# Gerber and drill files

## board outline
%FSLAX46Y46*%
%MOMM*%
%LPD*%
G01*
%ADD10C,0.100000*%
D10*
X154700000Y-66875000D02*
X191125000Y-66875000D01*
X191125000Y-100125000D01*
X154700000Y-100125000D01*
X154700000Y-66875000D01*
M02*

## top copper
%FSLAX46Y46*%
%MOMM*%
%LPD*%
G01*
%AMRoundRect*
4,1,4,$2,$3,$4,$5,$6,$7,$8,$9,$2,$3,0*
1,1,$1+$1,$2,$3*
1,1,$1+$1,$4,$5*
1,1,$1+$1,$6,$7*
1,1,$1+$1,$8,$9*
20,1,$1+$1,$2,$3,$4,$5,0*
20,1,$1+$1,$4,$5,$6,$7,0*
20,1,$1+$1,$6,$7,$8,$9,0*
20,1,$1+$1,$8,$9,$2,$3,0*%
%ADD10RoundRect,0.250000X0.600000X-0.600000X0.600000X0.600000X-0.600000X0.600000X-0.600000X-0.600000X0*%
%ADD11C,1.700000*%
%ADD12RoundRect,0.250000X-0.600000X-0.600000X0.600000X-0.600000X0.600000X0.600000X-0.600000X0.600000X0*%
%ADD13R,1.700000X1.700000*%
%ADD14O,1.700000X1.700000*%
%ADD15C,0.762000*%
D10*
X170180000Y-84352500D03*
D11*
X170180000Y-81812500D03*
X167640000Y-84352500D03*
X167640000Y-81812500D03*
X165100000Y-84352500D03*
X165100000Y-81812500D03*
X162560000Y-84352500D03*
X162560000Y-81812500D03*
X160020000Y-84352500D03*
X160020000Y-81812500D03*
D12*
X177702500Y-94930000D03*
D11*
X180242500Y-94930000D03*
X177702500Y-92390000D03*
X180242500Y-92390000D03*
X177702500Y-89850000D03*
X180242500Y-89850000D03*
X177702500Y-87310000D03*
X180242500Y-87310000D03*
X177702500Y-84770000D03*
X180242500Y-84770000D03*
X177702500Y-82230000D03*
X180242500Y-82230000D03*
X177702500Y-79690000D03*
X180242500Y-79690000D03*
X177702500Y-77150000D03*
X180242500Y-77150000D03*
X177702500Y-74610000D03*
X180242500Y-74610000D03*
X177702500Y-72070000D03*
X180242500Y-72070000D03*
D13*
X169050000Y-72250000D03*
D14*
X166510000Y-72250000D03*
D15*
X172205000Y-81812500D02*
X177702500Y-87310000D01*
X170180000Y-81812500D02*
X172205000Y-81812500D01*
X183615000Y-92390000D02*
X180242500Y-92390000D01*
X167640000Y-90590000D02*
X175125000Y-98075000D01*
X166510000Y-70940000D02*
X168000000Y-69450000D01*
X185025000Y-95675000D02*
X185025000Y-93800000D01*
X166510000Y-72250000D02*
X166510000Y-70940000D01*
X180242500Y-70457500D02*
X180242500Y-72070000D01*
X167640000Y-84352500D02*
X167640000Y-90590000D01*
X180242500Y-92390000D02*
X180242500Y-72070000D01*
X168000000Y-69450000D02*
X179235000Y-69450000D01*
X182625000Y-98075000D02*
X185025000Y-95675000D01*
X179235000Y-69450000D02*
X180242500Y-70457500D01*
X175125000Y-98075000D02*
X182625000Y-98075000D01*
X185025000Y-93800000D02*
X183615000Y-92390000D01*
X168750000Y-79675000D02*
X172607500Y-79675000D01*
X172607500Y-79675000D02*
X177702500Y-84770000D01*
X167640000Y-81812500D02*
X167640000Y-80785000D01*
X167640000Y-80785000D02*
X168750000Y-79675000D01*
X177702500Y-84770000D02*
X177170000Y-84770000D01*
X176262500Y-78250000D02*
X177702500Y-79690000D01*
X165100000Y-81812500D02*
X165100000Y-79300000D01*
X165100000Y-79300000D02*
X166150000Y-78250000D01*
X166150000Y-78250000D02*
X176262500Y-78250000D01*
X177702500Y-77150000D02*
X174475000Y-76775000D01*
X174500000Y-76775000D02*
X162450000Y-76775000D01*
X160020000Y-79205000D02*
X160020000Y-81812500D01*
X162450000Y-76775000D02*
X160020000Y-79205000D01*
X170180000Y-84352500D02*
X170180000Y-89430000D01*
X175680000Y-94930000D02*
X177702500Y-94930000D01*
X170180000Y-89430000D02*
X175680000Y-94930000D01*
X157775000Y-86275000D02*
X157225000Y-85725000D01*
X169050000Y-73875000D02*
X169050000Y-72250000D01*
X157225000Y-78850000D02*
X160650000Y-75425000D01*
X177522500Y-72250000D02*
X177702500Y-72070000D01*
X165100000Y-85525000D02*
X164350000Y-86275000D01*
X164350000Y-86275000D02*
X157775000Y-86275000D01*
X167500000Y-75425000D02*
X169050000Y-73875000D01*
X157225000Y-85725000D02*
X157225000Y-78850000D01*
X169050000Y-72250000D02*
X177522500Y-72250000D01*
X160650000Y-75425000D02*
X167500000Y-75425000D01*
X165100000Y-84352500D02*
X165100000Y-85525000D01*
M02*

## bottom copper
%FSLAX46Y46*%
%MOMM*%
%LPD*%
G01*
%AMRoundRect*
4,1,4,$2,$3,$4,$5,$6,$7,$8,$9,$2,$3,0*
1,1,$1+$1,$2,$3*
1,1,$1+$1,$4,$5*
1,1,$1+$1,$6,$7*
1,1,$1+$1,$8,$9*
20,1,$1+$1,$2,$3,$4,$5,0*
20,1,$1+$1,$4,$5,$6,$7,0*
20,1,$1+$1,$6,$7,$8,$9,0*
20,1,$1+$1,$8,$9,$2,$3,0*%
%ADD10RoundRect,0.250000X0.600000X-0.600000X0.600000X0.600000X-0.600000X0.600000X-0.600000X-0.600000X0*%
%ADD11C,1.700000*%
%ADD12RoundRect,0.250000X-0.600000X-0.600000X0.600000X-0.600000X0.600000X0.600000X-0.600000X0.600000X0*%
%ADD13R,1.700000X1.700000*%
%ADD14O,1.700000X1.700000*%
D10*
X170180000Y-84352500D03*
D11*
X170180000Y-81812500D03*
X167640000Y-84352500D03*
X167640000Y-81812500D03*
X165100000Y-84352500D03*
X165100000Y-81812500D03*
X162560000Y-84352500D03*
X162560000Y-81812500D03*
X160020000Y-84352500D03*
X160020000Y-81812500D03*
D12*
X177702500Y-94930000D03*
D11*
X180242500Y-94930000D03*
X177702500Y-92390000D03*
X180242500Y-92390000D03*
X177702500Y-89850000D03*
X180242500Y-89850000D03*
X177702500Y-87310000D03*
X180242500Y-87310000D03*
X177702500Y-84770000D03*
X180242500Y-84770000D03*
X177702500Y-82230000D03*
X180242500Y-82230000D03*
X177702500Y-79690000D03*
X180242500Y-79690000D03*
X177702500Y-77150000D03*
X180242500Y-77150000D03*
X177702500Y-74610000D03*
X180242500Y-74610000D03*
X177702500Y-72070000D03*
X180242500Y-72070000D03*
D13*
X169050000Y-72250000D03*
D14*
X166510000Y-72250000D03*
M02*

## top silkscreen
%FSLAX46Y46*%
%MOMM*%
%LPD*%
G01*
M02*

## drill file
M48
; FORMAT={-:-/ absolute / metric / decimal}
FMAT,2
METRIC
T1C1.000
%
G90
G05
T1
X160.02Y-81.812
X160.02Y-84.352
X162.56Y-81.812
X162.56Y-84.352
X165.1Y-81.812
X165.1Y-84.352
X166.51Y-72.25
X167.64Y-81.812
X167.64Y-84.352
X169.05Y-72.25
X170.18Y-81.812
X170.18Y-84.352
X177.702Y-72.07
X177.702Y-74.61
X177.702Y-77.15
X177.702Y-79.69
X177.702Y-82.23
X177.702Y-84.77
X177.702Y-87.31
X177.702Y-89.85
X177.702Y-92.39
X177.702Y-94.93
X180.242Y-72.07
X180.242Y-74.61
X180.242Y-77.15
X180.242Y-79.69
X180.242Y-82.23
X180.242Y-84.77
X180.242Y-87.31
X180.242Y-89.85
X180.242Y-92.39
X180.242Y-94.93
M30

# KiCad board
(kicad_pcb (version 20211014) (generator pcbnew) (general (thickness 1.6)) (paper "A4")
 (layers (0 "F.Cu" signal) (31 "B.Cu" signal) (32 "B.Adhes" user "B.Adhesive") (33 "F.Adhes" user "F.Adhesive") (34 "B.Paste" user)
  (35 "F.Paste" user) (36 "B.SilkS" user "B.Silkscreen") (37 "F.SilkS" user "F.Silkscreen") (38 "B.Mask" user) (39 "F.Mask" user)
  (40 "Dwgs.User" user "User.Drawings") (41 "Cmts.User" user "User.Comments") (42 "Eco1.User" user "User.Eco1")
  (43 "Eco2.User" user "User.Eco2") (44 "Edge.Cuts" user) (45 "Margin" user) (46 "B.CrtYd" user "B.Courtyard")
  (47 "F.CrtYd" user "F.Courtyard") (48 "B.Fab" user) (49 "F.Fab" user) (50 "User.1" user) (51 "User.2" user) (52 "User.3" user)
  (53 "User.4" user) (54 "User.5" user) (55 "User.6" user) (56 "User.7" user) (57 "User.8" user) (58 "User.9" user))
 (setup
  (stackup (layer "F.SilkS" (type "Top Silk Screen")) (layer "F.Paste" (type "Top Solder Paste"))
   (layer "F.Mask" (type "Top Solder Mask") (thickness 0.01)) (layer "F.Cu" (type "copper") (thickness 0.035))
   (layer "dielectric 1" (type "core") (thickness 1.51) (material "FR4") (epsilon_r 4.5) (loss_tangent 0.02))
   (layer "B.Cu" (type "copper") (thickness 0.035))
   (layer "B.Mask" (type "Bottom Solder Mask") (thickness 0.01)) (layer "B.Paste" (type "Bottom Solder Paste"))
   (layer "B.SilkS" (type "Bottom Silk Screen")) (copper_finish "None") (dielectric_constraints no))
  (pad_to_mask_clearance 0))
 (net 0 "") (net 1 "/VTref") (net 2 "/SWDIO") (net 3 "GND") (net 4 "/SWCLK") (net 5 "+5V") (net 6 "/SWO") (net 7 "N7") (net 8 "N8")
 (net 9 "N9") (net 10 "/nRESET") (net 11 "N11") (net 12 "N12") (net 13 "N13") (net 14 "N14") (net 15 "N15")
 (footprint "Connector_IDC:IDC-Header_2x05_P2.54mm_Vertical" (layer "B.Cu") (at 170.18 84.3525 90)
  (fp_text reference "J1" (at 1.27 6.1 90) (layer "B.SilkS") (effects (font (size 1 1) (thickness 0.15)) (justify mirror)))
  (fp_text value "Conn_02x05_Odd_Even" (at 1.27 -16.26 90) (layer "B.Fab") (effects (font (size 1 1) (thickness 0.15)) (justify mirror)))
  (pad "1" thru_hole roundrect (at 0 0 90) (size 1.7 1.7) (drill 1) (layers *.Cu *.Mask) (roundrect_rratio 0.147059) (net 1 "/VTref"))
  (pad "2" thru_hole circle (at 2.54 0 90) (size 1.7 1.7) (drill 1) (layers *.Cu *.Mask) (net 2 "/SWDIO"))
  (pad "3" thru_hole circle (at 0 -2.54 90) (size 1.7 1.7) (drill 1) (layers *.Cu *.Mask) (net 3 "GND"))
  (pad "4" thru_hole circle (at 2.54 -2.54 90) (size 1.7 1.7) (drill 1) (layers *.Cu *.Mask) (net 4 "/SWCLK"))
  (pad "5" thru_hole circle (at 0 -5.08 90) (size 1.7 1.7) (drill 1) (layers *.Cu *.Mask) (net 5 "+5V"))
  (pad "6" thru_hole circle (at 2.54 -5.08 90) (size 1.7 1.7) (drill 1) (layers *.Cu *.Mask) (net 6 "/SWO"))
  (pad "7" thru_hole circle (at 0 -7.62 90) (size 1.7 1.7) (drill 1) (layers *.Cu *.Mask) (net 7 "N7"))
  (pad "8" thru_hole circle (at 2.54 -7.62 90) (size 1.7 1.7) (drill 1) (layers *.Cu *.Mask) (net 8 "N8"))
  (pad "9" thru_hole circle (at 0 -10.16 90) (size 1.7 1.7) (drill 1) (layers *.Cu *.Mask) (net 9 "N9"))
  (pad "10" thru_hole circle (at 2.54 -10.16 90) (size 1.7 1.7) (drill 1) (layers *.Cu *.Mask) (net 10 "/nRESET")))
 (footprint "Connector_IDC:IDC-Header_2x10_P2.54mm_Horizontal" (layer "B.Cu") (at 177.7025 94.93)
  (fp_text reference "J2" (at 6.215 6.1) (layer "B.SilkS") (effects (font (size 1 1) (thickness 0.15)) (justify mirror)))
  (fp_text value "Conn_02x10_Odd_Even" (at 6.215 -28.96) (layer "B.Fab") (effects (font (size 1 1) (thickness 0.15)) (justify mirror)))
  (pad "1" thru_hole roundrect (at 0 0) (size 1.7 1.7) (drill 1) (layers *.Cu *.Mask) (roundrect_rratio 0.1470588235) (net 1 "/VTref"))
  (pad "2" thru_hole circle (at 2.54 0) (size 1.7 1.7) (drill 1) (layers *.Cu *.Mask) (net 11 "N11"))
  (pad "3" thru_hole circle (at 0 -2.54) (size 1.7 1.7) (drill 1) (layers *.Cu *.Mask) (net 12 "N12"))
  (pad "4" thru_hole circle (at 2.54 -2.54) (size 1.7 1.7) (drill 1) (layers *.Cu *.Mask) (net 3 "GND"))
  (pad "5" thru_hole circle (at 0 -5.08) (size 1.7 1.7) (drill 1) (layers *.Cu *.Mask) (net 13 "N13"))
  (pad "6" thru_hole circle (at 2.54 -5.08) (size 1.7 1.7) (drill 1) (layers *.Cu *.Mask) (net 3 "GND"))
  (pad "7" thru_hole circle (at 0 -7.62) (size 1.7 1.7) (drill 1) (layers *.Cu *.Mask) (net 2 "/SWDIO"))
  (pad "8" thru_hole circle (at 2.54 -7.62) (size 1.7 1.7) (drill 1) (layers *.Cu *.Mask) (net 3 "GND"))
  (pad "9" thru_hole circle (at 0 -10.16) (size 1.7 1.7) (drill 1) (layers *.Cu *.Mask) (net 4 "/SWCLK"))
  (pad "10" thru_hole circle (at 2.54 -10.16) (size 1.7 1.7) (drill 1) (layers *.Cu *.Mask) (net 3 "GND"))
  (pad "11" thru_hole circle (at 0 -12.7) (size 1.7 1.7) (drill 1) (layers *.Cu *.Mask) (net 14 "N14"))
  (pad "12" thru_hole circle (at 2.54 -12.7) (size 1.7 1.7) (drill 1) (layers *.Cu *.Mask) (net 3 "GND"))
  (pad "13" thru_hole circle (at 0 -15.24) (size 1.7 1.7) (drill 1) (layers *.Cu *.Mask) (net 6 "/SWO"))
  (pad "14" thru_hole circle (at 2.54 -15.24) (size 1.7 1.7) (drill 1) (layers *.Cu *.Mask) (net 3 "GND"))
  (pad "15" thru_hole circle (at 0 -17.78) (size 1.7 1.7) (drill 1) (layers *.Cu *.Mask) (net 10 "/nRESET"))
  (pad "16" thru_hole circle (at 2.54 -17.78) (size 1.7 1.7) (drill 1) (layers *.Cu *.Mask) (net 3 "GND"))
  (pad "17" thru_hole circle (at 0 -20.32) (size 1.7 1.7) (drill 1) (layers *.Cu *.Mask) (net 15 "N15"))
  (pad "18" thru_hole circle (at 2.54 -20.32) (size 1.7 1.7) (drill 1) (layers *.Cu *.Mask) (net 3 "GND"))
  (pad "19" thru_hole circle (at 0 -22.86) (size 1.7 1.7) (drill 1) (layers *.Cu *.Mask) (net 5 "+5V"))
  (pad "20" thru_hole circle (at 2.54 -22.86) (size 1.7 1.7) (drill 1) (layers *.Cu *.Mask) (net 3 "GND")))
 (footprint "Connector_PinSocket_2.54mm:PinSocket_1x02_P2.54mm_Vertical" (layer "B.Cu") (at 169.05 72.25 90)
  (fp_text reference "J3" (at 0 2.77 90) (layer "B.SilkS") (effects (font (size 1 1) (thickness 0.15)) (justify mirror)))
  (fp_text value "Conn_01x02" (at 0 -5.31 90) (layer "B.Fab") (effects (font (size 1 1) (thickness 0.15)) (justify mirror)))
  (pad "1" thru_hole rect (at 0 0 90) (size 1.7 1.7) (drill 1) (layers *.Cu *.Mask) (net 5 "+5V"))
  (pad "2" thru_hole oval (at 0 -2.54 90) (size 1.7 1.7) (drill 1) (layers *.Cu *.Mask) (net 3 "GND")))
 (gr_rect (start 191.125 66.875) (end 154.7 100.125) (layer "Edge.Cuts") (width 0.1) (fill none))
 (segment (start 172.205 81.8125) (end 177.7025 87.31) (width 0.762) (layer "F.Cu") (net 2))
 (segment (start 170.18 81.8125) (end 172.205 81.8125) (width 0.762) (layer "F.Cu") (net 2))
 (segment (start 183.615 92.39) (end 180.2425 92.39) (width 0.762) (layer "F.Cu") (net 3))
 (segment (start 167.64 90.59) (end 175.125 98.075) (width 0.762) (layer "F.Cu") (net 3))
 (segment (start 166.51 70.94) (end 168 69.45) (width 0.762) (layer "F.Cu") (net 3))
 (segment (start 185.025 95.675) (end 185.025 93.8) (width 0.762) (layer "F.Cu") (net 3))
 (segment (start 166.51 72.25) (end 166.51 70.94) (width 0.762) (layer "F.Cu") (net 3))
 (segment (start 180.2425 70.4575) (end 180.2425 72.07) (width 0.762) (layer "F.Cu") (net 3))
 (segment (start 167.64 84.3525) (end 167.64 90.59) (width 0.762) (layer "F.Cu") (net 3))
 (segment (start 180.2425 92.39) (end 180.2425 72.07) (width 0.762) (layer "F.Cu") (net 3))
 (segment (start 168 69.45) (end 179.235 69.45) (width 0.762) (layer "F.Cu") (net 3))
 (segment (start 182.625 98.075) (end 185.025 95.675) (width 0.762) (layer "F.Cu") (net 3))
 (segment (start 179.235 69.45) (end 180.2425 70.4575) (width 0.762) (layer "F.Cu") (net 3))
 (segment (start 175.125 98.075) (end 182.625 98.075) (width 0.762) (layer "F.Cu") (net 3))
 (segment (start 185.025 93.8) (end 183.615 92.39) (width 0.762) (layer "F.Cu") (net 3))
 (segment (start 168.75 79.675) (end 172.6075 79.675) (width 0.762) (layer "F.Cu") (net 4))
 (segment (start 172.6075 79.675) (end 177.7025 84.77) (width 0.762) (layer "F.Cu") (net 4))
 (segment (start 167.64 81.8125) (end 167.64 80.785) (width 0.762) (layer "F.Cu") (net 4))
 (segment (start 167.64 80.785) (end 168.75 79.675) (width 0.762) (layer "F.Cu") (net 4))
 (segment (start 177.7025 84.77) (end 177.17 84.77) (width 0.762) (layer "F.Cu") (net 4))
 (segment (start 176.2625 78.25) (end 177.7025 79.69) (width 0.762) (layer "F.Cu") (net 6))
 (segment (start 165.1 81.8125) (end 165.1 79.3) (width 0.762) (layer "F.Cu") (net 6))
 (segment (start 165.1 79.3) (end 166.15 78.25) (width 0.762) (layer "F.Cu") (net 6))
 (segment (start 166.15 78.25) (end 176.2625 78.25) (width 0.762) (layer "F.Cu") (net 6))
 (segment (start 177.7025 77.15) (end 174.475 76.775) (width 0.762) (layer "F.Cu") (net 10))
 (segment (start 174.5 76.775) (end 162.45 76.775) (width 0.762) (layer "F.Cu") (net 10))
 (segment (start 160.02 79.205) (end 160.02 81.8125) (width 0.762) (layer "F.Cu") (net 10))
 (segment (start 162.45 76.775) (end 160.02 79.205) (width 0.762) (layer "F.Cu") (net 10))
 (segment (start 170.18 84.3525) (end 170.18 89.43) (width 0.762) (layer "F.Cu") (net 1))
 (segment (start 175.68 94.93) (end 177.7025 94.93) (width 0.762) (layer "F.Cu") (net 1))
 (segment (start 170.18 89.43) (end 175.68 94.93) (width 0.762) (layer "F.Cu") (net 1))
 (segment (start 157.775 86.275) (end 157.225 85.725) (width 0.762) (layer "F.Cu") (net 5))
 (segment (start 169.05 73.875) (end 169.05 72.25) (width 0.762) (layer "F.Cu") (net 5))
 (segment (start 157.225 78.85) (end 160.65 75.425) (width 0.762) (layer "F.Cu") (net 5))
 (segment (start 177.5225 72.25) (end 177.7025 72.07) (width 0.762) (layer "F.Cu") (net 5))
 (segment (start 165.1 85.525) (end 164.35 86.275) (width 0.762) (layer "F.Cu") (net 5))
 (segment (start 164.35 86.275) (end 157.775 86.275) (width 0.762) (layer "F.Cu") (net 5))
 (segment (start 167.5 75.425) (end 169.05 73.875) (width 0.762) (layer "F.Cu") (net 5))
 (segment (start 157.225 85.725) (end 157.225 78.85) (width 0.762) (layer "F.Cu") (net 5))
 (segment (start 169.05 72.25) (end 177.5225 72.25) (width 0.762) (layer "F.Cu") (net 5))
 (segment (start 160.65 75.425) (end 167.5 75.425) (width 0.762) (layer "F.Cu") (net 5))
 (segment (start 165.1 84.3525) (end 165.1 85.525) (width 0.762) (layer "F.Cu") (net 5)))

